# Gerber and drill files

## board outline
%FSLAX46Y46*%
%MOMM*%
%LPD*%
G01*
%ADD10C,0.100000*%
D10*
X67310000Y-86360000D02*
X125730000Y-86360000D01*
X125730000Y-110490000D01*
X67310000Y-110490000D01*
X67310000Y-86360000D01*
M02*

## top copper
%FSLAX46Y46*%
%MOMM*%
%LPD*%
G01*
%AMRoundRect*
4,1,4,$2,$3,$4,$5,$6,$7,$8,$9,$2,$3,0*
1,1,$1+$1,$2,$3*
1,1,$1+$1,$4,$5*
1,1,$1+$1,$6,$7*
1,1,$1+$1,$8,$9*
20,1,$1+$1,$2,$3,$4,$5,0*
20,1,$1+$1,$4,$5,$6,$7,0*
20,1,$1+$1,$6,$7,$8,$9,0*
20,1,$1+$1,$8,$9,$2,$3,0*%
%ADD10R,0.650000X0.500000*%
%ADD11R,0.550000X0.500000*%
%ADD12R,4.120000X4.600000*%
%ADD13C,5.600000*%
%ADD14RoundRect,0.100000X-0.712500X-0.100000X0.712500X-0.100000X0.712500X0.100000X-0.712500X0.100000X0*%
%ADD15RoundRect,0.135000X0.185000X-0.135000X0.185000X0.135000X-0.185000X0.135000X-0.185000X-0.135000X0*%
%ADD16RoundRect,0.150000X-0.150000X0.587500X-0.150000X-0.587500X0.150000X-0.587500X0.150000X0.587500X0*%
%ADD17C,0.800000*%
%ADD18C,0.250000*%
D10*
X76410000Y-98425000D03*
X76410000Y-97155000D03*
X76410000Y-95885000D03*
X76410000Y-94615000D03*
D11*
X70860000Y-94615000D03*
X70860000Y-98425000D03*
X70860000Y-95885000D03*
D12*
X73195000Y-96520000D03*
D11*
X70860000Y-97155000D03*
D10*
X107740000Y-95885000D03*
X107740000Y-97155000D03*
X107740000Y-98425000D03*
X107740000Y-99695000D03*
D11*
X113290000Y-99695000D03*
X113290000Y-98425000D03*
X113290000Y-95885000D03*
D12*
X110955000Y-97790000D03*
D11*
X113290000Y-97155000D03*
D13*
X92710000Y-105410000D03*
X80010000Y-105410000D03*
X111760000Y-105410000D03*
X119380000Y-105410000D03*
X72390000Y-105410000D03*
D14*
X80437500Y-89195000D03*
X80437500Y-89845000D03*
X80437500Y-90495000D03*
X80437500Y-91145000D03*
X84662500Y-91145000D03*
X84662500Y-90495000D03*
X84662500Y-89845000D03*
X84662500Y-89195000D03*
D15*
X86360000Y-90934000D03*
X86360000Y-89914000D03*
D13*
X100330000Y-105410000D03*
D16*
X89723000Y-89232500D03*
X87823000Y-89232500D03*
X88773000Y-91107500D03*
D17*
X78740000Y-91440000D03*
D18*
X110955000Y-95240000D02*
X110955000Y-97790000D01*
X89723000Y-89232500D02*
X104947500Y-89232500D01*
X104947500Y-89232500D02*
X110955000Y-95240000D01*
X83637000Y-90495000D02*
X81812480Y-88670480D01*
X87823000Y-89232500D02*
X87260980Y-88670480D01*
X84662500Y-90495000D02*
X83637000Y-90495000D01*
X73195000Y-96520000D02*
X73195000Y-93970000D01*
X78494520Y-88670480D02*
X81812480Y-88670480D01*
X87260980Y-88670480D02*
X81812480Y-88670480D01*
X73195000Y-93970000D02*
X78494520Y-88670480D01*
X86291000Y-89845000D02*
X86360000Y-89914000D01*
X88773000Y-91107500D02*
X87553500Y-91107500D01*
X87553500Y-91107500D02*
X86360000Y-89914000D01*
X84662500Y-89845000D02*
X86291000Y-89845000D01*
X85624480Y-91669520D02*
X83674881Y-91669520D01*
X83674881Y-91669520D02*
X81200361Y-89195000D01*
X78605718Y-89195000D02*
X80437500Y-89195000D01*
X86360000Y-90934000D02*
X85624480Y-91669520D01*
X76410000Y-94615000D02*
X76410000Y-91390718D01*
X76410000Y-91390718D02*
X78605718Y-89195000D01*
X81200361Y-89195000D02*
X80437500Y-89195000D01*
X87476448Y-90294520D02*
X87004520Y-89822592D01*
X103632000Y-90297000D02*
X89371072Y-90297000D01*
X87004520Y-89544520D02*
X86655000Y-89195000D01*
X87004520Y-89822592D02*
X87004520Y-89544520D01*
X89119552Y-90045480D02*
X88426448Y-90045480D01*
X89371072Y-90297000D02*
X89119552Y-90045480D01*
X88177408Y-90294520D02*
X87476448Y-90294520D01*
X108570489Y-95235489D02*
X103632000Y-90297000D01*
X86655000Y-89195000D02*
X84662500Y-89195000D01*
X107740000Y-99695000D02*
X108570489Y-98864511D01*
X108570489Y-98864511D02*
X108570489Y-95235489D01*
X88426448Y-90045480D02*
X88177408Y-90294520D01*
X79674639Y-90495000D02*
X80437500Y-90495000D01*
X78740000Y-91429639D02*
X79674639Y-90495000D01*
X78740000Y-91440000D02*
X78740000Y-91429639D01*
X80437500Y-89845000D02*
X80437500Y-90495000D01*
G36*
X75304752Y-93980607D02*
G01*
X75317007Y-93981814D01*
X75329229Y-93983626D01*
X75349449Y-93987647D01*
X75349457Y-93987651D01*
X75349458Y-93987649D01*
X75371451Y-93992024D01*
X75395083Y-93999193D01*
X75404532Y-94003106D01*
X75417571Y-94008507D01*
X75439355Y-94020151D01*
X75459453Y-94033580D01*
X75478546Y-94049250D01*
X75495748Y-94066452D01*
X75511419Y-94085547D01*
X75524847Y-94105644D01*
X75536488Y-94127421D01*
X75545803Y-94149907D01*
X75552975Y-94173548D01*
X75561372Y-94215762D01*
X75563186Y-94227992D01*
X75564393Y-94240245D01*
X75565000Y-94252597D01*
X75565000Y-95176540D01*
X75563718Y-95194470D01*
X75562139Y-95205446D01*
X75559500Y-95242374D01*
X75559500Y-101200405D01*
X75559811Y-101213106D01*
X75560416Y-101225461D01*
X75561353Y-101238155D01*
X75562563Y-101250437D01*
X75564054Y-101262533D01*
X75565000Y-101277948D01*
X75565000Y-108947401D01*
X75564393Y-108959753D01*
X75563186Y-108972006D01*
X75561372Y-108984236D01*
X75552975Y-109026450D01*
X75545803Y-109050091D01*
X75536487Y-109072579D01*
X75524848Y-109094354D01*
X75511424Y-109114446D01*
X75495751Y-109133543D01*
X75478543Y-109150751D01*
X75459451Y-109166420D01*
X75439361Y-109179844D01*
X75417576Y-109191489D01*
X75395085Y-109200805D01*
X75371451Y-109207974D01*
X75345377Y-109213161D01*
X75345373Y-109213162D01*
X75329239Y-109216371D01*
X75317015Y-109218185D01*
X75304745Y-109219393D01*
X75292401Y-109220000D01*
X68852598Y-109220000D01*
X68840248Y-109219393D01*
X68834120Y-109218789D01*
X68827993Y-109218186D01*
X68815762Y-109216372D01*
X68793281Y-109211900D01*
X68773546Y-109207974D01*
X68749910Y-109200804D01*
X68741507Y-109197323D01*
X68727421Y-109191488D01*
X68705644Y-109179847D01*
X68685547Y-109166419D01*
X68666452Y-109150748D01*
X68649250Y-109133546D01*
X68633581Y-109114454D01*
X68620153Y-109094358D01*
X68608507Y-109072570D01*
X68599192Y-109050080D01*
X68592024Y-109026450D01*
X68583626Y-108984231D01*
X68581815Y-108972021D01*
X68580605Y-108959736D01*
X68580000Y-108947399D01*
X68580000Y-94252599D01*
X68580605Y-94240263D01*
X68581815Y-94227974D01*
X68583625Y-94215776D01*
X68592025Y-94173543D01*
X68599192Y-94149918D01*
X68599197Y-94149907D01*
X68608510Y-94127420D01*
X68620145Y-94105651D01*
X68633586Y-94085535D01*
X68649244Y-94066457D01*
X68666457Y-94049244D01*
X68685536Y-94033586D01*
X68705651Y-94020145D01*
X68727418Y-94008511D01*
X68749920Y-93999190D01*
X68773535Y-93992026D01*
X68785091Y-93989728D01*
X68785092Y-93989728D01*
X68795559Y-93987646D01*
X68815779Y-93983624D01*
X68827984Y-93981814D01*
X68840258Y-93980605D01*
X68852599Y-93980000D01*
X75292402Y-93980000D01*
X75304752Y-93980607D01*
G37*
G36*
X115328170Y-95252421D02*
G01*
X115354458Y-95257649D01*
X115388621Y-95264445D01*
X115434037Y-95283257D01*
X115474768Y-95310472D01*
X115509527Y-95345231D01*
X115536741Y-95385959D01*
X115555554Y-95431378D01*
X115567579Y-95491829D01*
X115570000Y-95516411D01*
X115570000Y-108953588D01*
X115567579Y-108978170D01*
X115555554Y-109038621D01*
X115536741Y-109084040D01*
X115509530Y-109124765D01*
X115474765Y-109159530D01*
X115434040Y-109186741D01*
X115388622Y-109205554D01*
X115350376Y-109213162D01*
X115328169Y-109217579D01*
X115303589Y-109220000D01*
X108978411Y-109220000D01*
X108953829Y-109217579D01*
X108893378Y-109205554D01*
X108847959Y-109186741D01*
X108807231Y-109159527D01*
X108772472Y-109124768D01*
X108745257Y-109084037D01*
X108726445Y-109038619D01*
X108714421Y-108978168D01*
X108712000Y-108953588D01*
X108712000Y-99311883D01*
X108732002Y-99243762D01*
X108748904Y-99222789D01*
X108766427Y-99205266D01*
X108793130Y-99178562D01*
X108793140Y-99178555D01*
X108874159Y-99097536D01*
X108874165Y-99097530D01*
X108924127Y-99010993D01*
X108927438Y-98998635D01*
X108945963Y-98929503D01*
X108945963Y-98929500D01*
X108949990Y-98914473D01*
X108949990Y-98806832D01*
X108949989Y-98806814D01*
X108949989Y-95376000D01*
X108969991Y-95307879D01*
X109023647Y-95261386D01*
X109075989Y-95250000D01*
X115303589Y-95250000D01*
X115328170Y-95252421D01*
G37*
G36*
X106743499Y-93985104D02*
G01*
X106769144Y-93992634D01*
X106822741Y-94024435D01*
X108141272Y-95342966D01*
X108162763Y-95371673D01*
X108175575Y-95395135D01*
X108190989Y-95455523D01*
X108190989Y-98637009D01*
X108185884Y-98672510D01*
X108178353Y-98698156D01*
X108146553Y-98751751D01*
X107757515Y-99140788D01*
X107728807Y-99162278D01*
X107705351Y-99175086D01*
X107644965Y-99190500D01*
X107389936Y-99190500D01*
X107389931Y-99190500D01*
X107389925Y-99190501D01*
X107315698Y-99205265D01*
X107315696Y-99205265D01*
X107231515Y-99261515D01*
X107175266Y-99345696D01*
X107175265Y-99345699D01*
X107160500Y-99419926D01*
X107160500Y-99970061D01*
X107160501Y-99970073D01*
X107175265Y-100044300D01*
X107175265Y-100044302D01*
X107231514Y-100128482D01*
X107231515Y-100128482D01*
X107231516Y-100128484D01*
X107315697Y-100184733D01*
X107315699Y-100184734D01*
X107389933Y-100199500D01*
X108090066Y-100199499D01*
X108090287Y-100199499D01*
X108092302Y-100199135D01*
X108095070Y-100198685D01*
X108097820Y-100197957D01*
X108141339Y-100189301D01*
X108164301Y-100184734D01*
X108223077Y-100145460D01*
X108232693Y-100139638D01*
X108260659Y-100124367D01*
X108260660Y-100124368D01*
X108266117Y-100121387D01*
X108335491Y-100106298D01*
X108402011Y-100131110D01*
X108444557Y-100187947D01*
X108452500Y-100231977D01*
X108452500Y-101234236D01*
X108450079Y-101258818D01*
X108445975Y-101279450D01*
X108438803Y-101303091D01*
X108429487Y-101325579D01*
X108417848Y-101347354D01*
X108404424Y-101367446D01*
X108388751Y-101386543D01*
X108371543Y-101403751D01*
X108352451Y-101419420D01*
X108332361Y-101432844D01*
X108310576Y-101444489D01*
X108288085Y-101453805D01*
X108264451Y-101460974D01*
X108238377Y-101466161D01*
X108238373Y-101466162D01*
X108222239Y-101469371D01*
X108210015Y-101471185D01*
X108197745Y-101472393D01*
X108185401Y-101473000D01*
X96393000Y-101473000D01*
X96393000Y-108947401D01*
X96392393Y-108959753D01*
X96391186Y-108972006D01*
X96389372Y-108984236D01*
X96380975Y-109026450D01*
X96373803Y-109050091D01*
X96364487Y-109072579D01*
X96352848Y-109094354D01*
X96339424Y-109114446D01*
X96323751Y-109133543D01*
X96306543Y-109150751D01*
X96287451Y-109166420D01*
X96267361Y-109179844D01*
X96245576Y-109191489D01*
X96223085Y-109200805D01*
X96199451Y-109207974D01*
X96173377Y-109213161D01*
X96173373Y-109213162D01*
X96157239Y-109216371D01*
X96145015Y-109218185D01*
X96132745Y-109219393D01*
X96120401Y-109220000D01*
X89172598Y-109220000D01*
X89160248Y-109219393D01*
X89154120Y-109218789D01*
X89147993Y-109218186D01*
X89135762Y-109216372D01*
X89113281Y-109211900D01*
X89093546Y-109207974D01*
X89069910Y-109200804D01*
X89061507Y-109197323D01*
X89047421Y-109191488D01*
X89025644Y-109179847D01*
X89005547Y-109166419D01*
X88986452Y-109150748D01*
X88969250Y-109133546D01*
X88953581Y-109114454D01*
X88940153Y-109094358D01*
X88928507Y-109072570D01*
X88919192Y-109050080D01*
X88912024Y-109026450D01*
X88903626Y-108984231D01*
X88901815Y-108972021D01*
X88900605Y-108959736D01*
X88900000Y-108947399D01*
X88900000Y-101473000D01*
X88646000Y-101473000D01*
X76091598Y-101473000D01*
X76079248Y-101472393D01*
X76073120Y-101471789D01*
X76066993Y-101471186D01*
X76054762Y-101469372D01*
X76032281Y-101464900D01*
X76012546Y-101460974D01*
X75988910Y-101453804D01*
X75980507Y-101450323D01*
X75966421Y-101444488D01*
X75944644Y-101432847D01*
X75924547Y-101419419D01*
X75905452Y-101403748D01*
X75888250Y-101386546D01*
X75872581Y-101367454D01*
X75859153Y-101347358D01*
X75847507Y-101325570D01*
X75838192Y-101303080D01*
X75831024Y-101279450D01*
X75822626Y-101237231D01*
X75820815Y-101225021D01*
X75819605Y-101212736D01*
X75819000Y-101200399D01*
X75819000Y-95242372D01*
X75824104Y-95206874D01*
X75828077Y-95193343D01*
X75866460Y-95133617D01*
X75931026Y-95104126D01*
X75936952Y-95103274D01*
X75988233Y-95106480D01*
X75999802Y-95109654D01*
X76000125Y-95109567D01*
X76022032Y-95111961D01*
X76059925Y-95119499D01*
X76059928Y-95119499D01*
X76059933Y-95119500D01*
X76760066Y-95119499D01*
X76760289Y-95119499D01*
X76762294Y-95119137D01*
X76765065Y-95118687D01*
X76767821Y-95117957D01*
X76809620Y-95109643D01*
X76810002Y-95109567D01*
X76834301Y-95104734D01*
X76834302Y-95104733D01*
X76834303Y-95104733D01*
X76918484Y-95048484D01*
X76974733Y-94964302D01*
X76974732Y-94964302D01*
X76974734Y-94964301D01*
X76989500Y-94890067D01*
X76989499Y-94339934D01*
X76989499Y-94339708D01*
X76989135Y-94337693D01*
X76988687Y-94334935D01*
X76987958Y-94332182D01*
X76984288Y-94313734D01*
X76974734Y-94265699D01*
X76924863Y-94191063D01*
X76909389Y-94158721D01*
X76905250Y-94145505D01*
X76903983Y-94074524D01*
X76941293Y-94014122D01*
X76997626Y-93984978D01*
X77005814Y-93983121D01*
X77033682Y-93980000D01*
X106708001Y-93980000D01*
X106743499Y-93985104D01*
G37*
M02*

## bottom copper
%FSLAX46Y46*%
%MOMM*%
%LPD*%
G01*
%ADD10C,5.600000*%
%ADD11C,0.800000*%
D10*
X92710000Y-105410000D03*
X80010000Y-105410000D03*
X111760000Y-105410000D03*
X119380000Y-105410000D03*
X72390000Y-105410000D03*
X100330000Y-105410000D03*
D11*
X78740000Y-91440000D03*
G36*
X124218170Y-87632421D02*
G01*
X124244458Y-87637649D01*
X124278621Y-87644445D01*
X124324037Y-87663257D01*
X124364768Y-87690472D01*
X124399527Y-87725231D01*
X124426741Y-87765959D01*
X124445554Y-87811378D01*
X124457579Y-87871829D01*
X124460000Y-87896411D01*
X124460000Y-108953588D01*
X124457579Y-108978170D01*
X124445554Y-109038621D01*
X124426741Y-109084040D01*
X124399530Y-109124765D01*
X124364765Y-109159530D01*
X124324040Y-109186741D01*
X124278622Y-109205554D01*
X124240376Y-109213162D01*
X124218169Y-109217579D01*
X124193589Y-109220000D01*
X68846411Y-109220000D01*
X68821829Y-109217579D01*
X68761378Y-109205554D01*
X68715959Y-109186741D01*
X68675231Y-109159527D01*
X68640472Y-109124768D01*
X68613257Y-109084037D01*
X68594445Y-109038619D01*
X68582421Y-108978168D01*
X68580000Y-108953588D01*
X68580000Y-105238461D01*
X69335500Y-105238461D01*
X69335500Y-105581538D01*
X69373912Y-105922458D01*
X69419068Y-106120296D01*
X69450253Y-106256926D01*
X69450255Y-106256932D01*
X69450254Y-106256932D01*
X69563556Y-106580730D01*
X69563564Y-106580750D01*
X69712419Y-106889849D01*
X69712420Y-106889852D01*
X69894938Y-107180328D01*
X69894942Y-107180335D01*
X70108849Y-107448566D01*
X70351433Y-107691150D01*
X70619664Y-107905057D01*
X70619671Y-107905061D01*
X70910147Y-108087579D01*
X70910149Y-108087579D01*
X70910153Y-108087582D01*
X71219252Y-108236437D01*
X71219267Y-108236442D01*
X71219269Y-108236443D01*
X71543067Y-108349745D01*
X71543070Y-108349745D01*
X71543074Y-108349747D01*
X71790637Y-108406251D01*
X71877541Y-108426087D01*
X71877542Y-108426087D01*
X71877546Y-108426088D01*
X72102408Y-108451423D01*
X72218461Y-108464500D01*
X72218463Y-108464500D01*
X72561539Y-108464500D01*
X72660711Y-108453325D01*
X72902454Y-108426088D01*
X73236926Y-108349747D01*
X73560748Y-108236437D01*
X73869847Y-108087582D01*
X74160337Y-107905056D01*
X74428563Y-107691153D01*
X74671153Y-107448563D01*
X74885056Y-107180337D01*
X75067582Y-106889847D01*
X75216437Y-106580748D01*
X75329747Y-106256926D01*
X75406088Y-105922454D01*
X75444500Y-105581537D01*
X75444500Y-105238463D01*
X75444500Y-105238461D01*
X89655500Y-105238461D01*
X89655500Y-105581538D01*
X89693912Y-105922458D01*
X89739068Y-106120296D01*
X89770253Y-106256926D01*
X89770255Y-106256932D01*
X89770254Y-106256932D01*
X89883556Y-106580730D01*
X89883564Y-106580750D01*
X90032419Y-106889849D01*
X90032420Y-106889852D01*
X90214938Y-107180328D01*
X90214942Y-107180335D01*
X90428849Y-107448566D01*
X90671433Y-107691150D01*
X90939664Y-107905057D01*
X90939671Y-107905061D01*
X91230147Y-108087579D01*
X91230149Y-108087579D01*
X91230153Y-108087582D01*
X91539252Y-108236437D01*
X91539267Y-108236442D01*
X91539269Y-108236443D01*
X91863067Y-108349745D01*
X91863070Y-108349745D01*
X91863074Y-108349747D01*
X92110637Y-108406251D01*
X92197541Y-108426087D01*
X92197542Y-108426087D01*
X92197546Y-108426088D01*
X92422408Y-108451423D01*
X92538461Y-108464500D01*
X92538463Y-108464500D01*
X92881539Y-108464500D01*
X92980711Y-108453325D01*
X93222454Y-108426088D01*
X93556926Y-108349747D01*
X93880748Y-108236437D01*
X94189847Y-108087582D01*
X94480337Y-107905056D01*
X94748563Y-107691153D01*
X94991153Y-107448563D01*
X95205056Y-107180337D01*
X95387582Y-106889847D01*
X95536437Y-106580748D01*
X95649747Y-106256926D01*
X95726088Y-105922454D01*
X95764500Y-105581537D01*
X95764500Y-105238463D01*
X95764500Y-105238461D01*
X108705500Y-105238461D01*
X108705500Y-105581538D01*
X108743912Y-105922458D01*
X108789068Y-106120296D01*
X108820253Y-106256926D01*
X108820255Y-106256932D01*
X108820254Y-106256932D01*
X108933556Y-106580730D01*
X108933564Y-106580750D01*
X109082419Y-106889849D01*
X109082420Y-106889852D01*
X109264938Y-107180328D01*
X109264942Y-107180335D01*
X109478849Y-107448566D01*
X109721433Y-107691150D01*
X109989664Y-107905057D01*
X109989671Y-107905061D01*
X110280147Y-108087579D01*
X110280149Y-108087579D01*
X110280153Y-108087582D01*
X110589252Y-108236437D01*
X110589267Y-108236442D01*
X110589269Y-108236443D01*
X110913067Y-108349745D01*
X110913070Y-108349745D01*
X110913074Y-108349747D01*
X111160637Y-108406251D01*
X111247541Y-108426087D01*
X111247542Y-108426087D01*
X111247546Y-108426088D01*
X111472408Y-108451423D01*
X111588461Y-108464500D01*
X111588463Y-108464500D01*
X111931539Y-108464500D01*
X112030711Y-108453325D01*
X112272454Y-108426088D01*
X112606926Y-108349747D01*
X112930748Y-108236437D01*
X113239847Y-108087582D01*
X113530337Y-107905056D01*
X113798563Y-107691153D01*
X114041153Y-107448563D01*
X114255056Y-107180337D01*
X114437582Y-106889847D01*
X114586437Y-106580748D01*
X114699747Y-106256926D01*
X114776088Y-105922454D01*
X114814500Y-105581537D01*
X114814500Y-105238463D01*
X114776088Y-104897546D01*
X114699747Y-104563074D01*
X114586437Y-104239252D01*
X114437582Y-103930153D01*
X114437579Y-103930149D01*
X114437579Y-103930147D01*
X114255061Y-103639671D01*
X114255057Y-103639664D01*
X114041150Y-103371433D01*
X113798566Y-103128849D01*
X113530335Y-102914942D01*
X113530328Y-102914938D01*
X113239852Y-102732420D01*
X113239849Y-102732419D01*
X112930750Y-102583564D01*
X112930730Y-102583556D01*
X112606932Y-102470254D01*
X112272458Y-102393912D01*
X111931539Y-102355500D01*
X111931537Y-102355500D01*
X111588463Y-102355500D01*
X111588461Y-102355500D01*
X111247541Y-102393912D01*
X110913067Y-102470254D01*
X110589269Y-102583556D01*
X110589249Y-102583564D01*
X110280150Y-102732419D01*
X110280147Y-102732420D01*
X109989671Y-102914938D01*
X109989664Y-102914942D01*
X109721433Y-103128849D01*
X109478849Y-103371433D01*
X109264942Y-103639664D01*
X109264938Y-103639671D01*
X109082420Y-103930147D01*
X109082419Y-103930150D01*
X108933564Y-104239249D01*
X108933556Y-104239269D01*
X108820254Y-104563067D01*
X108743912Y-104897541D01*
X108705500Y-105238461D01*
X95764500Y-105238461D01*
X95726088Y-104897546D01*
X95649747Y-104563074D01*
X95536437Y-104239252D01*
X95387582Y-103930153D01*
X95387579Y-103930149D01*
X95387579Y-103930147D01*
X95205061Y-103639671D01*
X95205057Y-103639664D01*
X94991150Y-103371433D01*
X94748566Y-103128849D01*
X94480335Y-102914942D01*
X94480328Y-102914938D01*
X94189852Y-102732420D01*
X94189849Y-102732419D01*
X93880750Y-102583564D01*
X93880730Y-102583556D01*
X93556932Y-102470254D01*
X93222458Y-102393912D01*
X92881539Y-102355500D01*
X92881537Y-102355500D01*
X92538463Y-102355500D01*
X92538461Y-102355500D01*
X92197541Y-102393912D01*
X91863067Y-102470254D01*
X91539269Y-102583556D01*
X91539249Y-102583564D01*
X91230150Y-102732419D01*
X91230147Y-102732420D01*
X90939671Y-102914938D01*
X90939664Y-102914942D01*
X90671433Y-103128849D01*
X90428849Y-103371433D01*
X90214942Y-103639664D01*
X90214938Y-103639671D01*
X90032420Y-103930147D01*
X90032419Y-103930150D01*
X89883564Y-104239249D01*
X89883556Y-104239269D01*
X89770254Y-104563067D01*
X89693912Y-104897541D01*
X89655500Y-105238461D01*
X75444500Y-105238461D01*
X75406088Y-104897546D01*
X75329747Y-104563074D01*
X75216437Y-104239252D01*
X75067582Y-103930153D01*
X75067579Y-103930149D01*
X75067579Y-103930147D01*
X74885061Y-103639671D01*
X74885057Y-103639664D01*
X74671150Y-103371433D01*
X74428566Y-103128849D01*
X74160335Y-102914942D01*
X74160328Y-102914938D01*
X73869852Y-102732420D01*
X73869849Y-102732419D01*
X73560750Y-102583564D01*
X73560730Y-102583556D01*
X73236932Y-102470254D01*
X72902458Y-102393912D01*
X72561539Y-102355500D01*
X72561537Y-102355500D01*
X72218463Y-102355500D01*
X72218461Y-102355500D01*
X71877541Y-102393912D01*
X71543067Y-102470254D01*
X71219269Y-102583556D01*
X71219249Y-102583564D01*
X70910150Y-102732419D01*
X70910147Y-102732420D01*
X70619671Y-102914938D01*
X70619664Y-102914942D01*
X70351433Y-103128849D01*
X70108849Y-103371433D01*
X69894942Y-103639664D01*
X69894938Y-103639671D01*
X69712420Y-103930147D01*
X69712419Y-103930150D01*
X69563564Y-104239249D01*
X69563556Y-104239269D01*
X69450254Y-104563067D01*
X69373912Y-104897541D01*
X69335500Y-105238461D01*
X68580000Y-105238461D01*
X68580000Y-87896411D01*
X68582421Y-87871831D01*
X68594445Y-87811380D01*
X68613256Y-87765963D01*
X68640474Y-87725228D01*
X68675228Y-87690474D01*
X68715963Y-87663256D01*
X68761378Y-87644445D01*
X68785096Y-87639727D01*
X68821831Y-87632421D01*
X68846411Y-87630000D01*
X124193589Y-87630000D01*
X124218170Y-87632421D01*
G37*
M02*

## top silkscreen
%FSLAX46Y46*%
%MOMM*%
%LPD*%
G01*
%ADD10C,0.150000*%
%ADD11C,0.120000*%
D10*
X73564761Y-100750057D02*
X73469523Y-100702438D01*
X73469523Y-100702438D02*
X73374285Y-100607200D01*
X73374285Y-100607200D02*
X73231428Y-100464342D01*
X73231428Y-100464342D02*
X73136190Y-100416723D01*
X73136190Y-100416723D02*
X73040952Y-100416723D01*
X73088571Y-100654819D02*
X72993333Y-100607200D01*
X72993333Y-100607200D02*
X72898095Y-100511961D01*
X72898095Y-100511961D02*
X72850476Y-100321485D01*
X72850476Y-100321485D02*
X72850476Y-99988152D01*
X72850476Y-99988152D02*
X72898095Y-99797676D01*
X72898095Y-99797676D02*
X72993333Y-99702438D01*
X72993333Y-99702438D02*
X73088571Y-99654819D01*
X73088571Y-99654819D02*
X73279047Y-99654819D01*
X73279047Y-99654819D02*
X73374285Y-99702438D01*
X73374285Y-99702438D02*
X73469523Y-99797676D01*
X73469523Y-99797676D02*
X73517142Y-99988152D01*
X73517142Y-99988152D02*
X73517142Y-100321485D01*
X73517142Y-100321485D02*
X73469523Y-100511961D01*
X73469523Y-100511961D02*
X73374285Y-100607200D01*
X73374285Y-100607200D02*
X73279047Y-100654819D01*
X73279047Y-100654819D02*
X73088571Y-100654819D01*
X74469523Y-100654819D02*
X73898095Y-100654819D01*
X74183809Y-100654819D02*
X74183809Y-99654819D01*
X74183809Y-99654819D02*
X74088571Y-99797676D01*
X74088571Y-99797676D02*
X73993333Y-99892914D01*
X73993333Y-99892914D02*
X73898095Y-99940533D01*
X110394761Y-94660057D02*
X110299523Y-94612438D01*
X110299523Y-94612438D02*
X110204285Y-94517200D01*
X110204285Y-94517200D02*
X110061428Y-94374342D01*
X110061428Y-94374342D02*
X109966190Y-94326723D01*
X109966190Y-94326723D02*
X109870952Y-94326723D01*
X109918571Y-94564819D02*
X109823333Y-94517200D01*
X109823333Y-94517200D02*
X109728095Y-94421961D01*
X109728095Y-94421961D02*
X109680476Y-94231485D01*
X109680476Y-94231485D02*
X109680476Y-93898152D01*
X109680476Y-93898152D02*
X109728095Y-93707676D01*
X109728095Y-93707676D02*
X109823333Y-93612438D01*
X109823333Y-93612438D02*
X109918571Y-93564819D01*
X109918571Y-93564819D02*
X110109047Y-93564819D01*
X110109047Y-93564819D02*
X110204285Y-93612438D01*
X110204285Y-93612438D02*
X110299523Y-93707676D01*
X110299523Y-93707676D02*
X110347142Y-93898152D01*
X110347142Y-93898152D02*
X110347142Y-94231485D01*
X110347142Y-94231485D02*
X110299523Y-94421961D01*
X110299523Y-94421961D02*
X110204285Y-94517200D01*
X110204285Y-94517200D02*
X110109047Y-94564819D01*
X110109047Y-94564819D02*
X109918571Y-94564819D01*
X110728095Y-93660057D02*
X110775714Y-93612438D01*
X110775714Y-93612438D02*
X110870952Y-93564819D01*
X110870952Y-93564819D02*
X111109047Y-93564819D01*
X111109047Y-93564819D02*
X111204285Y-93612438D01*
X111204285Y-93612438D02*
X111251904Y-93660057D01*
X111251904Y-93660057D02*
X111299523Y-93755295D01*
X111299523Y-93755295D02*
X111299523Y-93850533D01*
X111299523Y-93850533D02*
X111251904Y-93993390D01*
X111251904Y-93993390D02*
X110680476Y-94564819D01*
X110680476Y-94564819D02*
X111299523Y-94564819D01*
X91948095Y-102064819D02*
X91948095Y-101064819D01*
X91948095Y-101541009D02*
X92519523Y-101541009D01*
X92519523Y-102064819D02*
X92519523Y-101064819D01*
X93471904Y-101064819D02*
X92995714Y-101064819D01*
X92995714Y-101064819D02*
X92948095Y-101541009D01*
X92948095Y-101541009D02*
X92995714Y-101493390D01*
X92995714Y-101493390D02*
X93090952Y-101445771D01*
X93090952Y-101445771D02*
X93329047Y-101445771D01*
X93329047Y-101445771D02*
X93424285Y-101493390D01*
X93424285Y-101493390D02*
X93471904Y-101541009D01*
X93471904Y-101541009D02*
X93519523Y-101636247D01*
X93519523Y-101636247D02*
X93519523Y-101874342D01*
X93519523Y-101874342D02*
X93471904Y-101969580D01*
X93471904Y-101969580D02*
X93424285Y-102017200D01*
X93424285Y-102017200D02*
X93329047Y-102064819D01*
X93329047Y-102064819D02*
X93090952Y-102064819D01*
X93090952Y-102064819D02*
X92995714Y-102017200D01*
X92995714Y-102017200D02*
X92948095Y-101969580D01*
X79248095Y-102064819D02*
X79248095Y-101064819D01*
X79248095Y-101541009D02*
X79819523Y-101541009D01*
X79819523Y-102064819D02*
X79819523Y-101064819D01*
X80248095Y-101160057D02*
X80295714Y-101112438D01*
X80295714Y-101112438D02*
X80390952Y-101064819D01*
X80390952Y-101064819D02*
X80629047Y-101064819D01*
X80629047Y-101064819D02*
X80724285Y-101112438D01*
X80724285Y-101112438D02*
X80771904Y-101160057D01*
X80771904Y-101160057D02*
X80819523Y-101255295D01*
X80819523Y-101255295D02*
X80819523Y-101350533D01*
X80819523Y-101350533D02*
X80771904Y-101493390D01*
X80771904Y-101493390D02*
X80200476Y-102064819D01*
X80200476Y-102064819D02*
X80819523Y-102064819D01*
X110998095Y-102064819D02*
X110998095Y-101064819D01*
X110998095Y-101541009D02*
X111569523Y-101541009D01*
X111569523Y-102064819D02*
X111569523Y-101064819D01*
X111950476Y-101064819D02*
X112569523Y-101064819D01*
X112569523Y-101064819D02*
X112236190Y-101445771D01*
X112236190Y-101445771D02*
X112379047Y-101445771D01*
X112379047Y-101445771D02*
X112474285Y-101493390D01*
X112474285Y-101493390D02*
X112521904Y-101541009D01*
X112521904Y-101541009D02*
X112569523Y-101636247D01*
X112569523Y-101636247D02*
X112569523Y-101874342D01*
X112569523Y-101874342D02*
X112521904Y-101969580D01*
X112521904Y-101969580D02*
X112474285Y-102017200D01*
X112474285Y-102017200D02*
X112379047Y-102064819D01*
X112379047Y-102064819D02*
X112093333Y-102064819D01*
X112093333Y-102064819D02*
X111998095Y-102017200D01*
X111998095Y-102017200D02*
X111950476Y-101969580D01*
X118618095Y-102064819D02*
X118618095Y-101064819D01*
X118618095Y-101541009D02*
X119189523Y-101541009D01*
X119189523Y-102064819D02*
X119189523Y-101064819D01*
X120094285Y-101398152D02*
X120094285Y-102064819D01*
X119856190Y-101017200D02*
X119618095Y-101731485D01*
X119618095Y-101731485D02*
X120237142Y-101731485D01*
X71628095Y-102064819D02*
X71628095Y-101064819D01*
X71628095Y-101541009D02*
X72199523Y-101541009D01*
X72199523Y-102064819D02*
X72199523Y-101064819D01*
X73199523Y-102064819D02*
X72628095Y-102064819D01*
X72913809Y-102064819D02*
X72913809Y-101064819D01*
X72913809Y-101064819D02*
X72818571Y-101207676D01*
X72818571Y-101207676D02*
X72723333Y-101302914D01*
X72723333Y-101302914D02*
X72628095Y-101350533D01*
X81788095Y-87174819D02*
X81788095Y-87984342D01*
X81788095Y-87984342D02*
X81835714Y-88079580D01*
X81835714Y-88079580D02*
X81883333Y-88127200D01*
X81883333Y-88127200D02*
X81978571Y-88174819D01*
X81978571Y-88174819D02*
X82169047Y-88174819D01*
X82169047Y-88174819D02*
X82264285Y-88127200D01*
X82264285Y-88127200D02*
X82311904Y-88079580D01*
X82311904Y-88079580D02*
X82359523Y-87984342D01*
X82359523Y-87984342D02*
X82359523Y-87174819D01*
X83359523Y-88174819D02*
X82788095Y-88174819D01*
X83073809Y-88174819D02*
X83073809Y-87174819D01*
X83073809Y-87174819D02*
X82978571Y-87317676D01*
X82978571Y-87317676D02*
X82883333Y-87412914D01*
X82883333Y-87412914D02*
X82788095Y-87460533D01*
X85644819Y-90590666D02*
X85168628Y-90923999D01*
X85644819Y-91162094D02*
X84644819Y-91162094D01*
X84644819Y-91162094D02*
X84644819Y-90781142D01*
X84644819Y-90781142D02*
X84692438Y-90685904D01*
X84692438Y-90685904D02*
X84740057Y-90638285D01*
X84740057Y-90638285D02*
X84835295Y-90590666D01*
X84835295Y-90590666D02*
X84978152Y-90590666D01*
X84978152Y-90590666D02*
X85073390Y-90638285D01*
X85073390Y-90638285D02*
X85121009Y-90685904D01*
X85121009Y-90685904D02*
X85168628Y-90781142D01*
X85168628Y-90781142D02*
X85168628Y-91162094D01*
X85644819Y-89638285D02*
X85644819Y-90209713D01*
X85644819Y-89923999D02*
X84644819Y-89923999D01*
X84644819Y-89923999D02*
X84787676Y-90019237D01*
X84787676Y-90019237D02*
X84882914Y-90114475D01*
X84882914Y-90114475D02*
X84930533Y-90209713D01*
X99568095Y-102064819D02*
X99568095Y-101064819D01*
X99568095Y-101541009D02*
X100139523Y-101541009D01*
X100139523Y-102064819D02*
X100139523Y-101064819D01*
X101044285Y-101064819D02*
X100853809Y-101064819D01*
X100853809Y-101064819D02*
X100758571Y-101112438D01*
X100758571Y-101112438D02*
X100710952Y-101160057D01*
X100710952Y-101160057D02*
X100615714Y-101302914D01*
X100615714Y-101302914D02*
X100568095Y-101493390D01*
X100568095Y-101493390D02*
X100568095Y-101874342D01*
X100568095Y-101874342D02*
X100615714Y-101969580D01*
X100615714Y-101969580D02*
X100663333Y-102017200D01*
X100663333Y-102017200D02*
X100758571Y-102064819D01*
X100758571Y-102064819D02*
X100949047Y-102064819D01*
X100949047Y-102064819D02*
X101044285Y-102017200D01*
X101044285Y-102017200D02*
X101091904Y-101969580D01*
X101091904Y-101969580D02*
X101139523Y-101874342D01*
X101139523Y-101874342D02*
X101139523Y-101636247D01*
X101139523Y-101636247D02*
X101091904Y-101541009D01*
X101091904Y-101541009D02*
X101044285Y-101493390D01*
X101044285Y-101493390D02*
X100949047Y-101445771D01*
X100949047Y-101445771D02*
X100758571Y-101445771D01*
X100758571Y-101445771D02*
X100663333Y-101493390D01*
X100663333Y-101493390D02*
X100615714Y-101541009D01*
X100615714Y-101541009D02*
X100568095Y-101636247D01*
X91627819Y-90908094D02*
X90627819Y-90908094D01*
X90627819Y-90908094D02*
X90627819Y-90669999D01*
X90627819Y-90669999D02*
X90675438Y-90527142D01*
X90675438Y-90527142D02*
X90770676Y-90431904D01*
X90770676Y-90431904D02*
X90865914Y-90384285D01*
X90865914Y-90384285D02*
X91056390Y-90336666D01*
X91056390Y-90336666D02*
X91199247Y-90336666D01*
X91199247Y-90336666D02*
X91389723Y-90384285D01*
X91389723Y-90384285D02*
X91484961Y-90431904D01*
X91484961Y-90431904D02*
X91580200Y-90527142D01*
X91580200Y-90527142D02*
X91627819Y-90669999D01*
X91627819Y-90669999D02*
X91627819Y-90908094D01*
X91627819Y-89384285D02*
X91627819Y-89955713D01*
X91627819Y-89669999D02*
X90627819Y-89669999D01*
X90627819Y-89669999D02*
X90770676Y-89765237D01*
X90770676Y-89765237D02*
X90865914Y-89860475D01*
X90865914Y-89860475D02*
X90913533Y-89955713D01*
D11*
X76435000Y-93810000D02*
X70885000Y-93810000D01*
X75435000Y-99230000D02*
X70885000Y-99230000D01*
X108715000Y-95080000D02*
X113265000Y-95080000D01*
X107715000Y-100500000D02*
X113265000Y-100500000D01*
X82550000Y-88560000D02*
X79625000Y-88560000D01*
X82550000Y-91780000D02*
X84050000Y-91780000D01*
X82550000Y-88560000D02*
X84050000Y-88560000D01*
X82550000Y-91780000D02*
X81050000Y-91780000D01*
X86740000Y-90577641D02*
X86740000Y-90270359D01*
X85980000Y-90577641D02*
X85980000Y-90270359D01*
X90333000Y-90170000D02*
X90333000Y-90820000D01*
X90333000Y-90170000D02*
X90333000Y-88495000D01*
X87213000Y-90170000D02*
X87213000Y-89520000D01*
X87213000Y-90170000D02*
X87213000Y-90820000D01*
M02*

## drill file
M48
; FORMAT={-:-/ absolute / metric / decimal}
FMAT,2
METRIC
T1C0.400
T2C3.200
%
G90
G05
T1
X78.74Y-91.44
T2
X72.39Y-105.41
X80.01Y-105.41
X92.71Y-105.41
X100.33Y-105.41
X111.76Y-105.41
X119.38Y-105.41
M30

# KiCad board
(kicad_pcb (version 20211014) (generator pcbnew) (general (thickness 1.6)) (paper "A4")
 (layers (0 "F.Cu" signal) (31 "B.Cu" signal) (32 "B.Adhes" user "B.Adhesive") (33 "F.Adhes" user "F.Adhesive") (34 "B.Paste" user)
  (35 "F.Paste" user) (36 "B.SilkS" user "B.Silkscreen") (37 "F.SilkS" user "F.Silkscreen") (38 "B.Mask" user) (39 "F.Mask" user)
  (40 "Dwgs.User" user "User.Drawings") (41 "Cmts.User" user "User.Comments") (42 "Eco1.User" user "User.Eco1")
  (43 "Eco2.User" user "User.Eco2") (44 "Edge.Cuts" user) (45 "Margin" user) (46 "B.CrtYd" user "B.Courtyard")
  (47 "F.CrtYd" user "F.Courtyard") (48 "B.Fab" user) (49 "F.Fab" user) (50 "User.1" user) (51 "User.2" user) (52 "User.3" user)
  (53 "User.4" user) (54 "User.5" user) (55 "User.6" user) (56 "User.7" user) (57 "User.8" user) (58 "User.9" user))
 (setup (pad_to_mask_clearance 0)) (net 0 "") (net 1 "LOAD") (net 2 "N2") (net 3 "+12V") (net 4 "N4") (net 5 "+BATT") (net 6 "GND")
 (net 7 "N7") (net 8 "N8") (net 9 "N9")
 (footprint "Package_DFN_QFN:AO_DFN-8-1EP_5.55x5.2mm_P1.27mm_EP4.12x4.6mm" (layer "F.Cu") (at 73.66 96.52 180)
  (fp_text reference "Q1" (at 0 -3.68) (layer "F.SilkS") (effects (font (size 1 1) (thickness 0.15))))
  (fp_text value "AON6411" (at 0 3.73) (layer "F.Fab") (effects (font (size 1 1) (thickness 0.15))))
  (fp_line (start -2.775 2.71) (end 2.775 2.71) (layer "F.SilkS") (width 0.12))
  (fp_line (start -1.775 -2.71) (end 2.775 -2.71) (layer "F.SilkS") (width 0.12))
  (pad "" smd rect (at -0.02 -1.65 90) (size 0.9 0.78) (layers "F.Paste"))
  (pad "" smd rect (at 0.96 1.65 90) (size 0.9 0.78) (layers "F.Paste"))
  (pad "" smd rect (at 0.96 0.55 90) (size 0.9 0.78) (layers "F.Paste"))
  (pad "" smd rect (at 1.94 -0.55 90) (size 0.9 0.78) (layers "F.Paste"))
  (pad "" smd rect (at 1.94 -1.65 90) (size 0.9 0.78) (layers "F.Paste"))
  (pad "" smd rect (at -1 1.65 90) (size 0.9 0.78) (layers "F.Paste"))
  (pad "" smd rect (at 0.96 -0.55 90) (size 0.9 0.78) (layers "F.Paste"))
  (pad "" smd rect (at -1 -0.55 90) (size 0.9 0.78) (layers "F.Paste"))
  (pad "" smd rect (at -1 0.55 90) (size 0.9 0.78) (layers "F.Paste"))
  (pad "" smd rect (at 1.94 0.55 90) (size 0.9 0.78) (layers "F.Paste"))
  (pad "" smd rect (at -0.02 1.65 90) (size 0.9 0.78) (layers "F.Paste"))
  (pad "" smd rect (at -0.02 -0.55 90) (size 0.9 0.78) (layers "F.Paste"))
  (pad "" smd rect (at 0.96 -1.65 90) (size 0.9 0.78) (layers "F.Paste"))
  (pad "" smd rect (at -1 -1.65 90) (size 0.9 0.78) (layers "F.Paste"))
  (pad "" smd rect (at 1.94 1.65 90) (size 0.9 0.78) (layers "F.Paste"))
  (pad "" smd rect (at -0.02 0.55 90) (size 0.9 0.78) (layers "F.Paste"))
  (pad "1" smd rect (at -2.75 -1.905 90) (size 0.5 0.65) (layers "F.Cu" "F.Paste" "F.Mask") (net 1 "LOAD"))
  (pad "2" smd rect (at -2.75 -0.635 90) (size 0.5 0.65) (layers "F.Cu" "F.Paste" "F.Mask") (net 1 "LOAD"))
  (pad "3" smd rect (at -2.75 0.635 90) (size 0.5 0.65) (layers "F.Cu" "F.Paste" "F.Mask") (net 1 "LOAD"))
  (pad "4" smd rect (at -2.75 1.905 90) (size 0.5 0.65) (layers "F.Cu" "F.Paste" "F.Mask") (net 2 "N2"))
  (pad "5" smd rect (at 2.8 1.905 90) (size 0.5 0.55) (layers "F.Cu" "F.Paste" "F.Mask") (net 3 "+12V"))
  (pad "5" smd rect (at 2.8 -1.905 90) (size 0.5 0.55) (layers "F.Cu" "F.Paste" "F.Mask") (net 3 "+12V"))
  (pad "5" smd rect (at 2.8 0.635 90) (size 0.5 0.55) (layers "F.Cu" "F.Paste" "F.Mask") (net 3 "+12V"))
  (pad "5" smd rect (at 0.465 0 90) (size 4.6 4.12) (layers "F.Cu" "F.Mask") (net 3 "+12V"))
  (pad "5" smd rect (at 2.8 -0.635 90) (size 0.5 0.55) (layers "F.Cu" "F.Paste" "F.Mask") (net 3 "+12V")))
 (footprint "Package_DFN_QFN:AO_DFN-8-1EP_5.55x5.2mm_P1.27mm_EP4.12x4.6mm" (layer "F.Cu") (at 110.49 97.79)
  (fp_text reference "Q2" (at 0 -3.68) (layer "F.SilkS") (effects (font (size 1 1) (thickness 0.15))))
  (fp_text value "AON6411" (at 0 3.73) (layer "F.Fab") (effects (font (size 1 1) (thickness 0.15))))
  (fp_line (start -1.775 -2.71) (end 2.775 -2.71) (layer "F.SilkS") (width 0.12))
  (fp_line (start -2.775 2.71) (end 2.775 2.71) (layer "F.SilkS") (width 0.12))
  (pad "" smd rect (at 1.94 1.65 270) (size 0.9 0.78) (layers "F.Paste"))
  (pad "" smd rect (at -0.02 1.65 270) (size 0.9 0.78) (layers "F.Paste"))
  (pad "" smd rect (at -1 -1.65 270) (size 0.9 0.78) (layers "F.Paste"))
  (pad "" smd rect (at -1 0.55 270) (size 0.9 0.78) (layers "F.Paste"))
  (pad "" smd rect (at 0.96 0.55 270) (size 0.9 0.78) (layers "F.Paste"))
  (pad "" smd rect (at 0.96 1.65 270) (size 0.9 0.78) (layers "F.Paste"))
  (pad "" smd rect (at 0.96 -1.65 270) (size 0.9 0.78) (layers "F.Paste"))
  (pad "" smd rect (at 0.96 -0.55 270) (size 0.9 0.78) (layers "F.Paste"))
  (pad "" smd rect (at 1.94 -1.65 270) (size 0.9 0.78) (layers "F.Paste"))
  (pad "" smd rect (at -0.02 -1.65 270) (size 0.9 0.78) (layers "F.Paste"))
  (pad "" smd rect (at -0.02 -0.55 270) (size 0.9 0.78) (layers "F.Paste"))
  (pad "" smd rect (at 1.94 0.55 270) (size 0.9 0.78) (layers "F.Paste"))
  (pad "" smd rect (at 1.94 -0.55 270) (size 0.9 0.78) (layers "F.Paste"))
  (pad "" smd rect (at -1 -0.55 270) (size 0.9 0.78) (layers "F.Paste"))
  (pad "" smd rect (at -0.02 0.55 270) (size 0.9 0.78) (layers "F.Paste"))
  (pad "" smd rect (at -1 1.65 270) (size 0.9 0.78) (layers "F.Paste"))
  (pad "1" smd rect (at -2.75 -1.905 270) (size 0.5 0.65) (layers "F.Cu" "F.Paste" "F.Mask") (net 1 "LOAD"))
  (pad "2" smd rect (at -2.75 -0.635 270) (size 0.5 0.65) (layers "F.Cu" "F.Paste" "F.Mask") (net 1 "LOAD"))
  (pad "3" smd rect (at -2.75 0.635 270) (size 0.5 0.65) (layers "F.Cu" "F.Paste" "F.Mask") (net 1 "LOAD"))
  (pad "4" smd rect (at -2.75 1.905 270) (size 0.5 0.65) (layers "F.Cu" "F.Paste" "F.Mask") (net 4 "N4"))
  (pad "5" smd rect (at 2.8 1.905 270) (size 0.5 0.55) (layers "F.Cu" "F.Paste" "F.Mask") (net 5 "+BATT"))
  (pad "5" smd rect (at 2.8 0.635 270) (size 0.5 0.55) (layers "F.Cu" "F.Paste" "F.Mask") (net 5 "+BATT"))
  (pad "5" smd rect (at 2.8 -1.905 270) (size 0.5 0.55) (layers "F.Cu" "F.Paste" "F.Mask") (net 5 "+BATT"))
  (pad "5" smd rect (at 0.465 0 270) (size 4.6 4.12) (layers "F.Cu" "F.Mask") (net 5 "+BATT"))
  (pad "5" smd rect (at 2.8 -0.635 270) (size 0.5 0.55) (layers "F.Cu" "F.Paste" "F.Mask") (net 5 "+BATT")))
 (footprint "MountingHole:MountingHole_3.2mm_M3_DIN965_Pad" (layer "F.Cu") (at 92.71 105.41)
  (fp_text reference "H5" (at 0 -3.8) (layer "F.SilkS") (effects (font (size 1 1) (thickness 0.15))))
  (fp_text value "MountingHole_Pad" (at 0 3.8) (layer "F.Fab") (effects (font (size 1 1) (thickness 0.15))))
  (pad "1" thru_hole circle (at 0 0) (size 5.6 5.6) (drill 3.2) (layers *.Cu *.Mask) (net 1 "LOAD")))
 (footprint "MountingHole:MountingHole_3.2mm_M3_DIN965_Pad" (layer "F.Cu") (at 80.01 105.41)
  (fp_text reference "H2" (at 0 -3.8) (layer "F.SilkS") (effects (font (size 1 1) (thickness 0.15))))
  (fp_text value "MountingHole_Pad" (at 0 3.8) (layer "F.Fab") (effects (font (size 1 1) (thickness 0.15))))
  (pad "1" thru_hole circle (at 0 0) (size 5.6 5.6) (drill 3.2) (layers *.Cu *.Mask) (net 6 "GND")))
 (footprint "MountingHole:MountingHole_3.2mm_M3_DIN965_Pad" (layer "F.Cu") (at 111.76 105.41)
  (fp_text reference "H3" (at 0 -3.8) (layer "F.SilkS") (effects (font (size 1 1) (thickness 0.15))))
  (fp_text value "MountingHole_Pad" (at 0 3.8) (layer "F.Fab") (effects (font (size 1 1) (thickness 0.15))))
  (pad "1" thru_hole circle (at 0 0) (size 5.6 5.6) (drill 3.2) (layers *.Cu *.Mask) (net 5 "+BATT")))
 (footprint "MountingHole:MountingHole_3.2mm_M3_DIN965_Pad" (layer "F.Cu") (at 119.38 105.41)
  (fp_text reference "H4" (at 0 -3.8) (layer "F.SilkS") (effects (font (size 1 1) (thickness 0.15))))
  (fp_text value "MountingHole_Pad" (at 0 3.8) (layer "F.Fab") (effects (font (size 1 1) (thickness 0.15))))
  (pad "1" thru_hole circle (at 0 0) (size 5.6 5.6) (drill 3.2) (layers *.Cu *.Mask) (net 6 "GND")))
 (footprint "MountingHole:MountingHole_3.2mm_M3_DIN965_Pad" (layer "F.Cu") (at 72.39 105.41)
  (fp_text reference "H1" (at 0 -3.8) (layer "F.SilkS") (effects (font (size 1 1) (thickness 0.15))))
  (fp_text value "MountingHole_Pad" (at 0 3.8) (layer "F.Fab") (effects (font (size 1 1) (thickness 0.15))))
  (pad "1" thru_hole circle (at 0 0) (size 5.6 5.6) (drill 3.2) (layers *.Cu *.Mask) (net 3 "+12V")))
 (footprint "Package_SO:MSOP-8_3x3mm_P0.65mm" (layer "F.Cu") (at 82.55 90.17)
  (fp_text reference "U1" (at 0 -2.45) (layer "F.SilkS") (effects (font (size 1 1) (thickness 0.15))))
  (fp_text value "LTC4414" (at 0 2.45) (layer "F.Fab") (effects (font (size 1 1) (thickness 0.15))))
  (fp_line (start 0 -1.61) (end -2.925 -1.61) (layer "F.SilkS") (width 0.12))
  (fp_line (start 0 1.61) (end 1.5 1.61) (layer "F.SilkS") (width 0.12))
  (fp_line (start 0 -1.61) (end 1.5 -1.61) (layer "F.SilkS") (width 0.12))
  (fp_line (start 0 1.61) (end -1.5 1.61) (layer "F.SilkS") (width 0.12))
  (pad "1" smd roundrect (at -2.1125 -0.975) (size 1.625 0.4) (layers "F.Cu" "F.Paste" "F.Mask") (roundrect_rratio 0.25) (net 2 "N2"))
  (pad "2" smd roundrect (at -2.1125 -0.325) (size 1.625 0.4) (layers "F.Cu" "F.Paste" "F.Mask") (roundrect_rratio 0.25) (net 6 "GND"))
  (pad "3" smd roundrect (at -2.1125 0.325) (size 1.625 0.4) (layers "F.Cu" "F.Paste" "F.Mask") (roundrect_rratio 0.25) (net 6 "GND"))
  (pad "4" smd roundrect (at -2.1125 0.975) (size 1.625 0.4) (layers "F.Cu" "F.Paste" "F.Mask") (roundrect_rratio 0.25) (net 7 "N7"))
  (pad "5" smd roundrect (at 2.1125 0.975) (size 1.625 0.4) (layers "F.Cu" "F.Paste" "F.Mask") (roundrect_rratio 0.25) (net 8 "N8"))
  (pad "6" smd roundrect (at 2.1125 0.325) (size 1.625 0.4) (layers "F.Cu" "F.Paste" "F.Mask") (roundrect_rratio 0.25) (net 3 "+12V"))
  (pad "7" smd roundrect (at 2.1125 -0.325) (size 1.625 0.4) (layers "F.Cu" "F.Paste" "F.Mask") (roundrect_rratio 0.25) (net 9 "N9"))
  (pad "8" smd roundrect (at 2.1125 -0.975) (size 1.625 0.4) (layers "F.Cu" "F.Paste" "F.Mask") (roundrect_rratio 0.25) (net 4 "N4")))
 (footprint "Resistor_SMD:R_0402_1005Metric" (layer "F.Cu") (at 86.36 90.424 90)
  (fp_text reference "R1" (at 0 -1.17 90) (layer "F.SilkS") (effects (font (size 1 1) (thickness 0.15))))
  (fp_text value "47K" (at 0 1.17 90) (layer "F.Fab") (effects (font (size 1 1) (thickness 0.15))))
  (fp_line (start -0.153641 0.38) (end 0.153641 0.38) (layer "F.SilkS") (width 0.12))
  (fp_line (start -0.153641 -0.38) (end 0.153641 -0.38) (layer "F.SilkS") (width 0.12))
  (pad "1" smd roundrect (at -0.51 0 90) (size 0.54 0.64) (layers "F.Cu" "F.Paste" "F.Mask") (roundrect_rratio 0.25) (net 2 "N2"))
  (pad "2" smd roundrect (at 0.51 0 90) (size 0.54 0.64) (layers "F.Cu" "F.Paste" "F.Mask") (roundrect_rratio 0.25) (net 9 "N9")))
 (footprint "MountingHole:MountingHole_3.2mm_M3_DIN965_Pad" (layer "F.Cu") (at 100.33 105.41)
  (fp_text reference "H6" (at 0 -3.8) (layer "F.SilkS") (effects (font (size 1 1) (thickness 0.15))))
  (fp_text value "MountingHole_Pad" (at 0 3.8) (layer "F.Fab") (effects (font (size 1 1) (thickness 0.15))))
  (pad "1" thru_hole circle (at 0 0) (size 5.6 5.6) (drill 3.2) (layers *.Cu *.Mask) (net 6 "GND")))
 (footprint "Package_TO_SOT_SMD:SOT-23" (layer "F.Cu") (at 88.773 90.17 -90)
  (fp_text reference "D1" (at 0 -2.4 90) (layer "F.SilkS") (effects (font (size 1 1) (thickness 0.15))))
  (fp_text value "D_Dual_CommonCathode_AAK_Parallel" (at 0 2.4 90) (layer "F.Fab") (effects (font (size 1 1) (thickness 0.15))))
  (fp_line (start 0 -1.56) (end 0.65 -1.56) (layer "F.SilkS") (width 0.12))
  (fp_line (start 0 -1.56) (end -1.675 -1.56) (layer "F.SilkS") (width 0.12))
  (fp_line (start 0 1.56) (end -0.65 1.56) (layer "F.SilkS") (width 0.12))
  (fp_line (start 0 1.56) (end 0.65 1.56) (layer "F.SilkS") (width 0.12))
  (pad "1" smd roundrect (at -0.9375 -0.95 270) (size 1.475 0.6) (layers "F.Cu" "F.Paste" "F.Mask") (roundrect_rratio 0.25) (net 5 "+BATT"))
  (pad "2" smd roundrect (at -0.9375 0.95 270) (size 1.475 0.6) (layers "F.Cu" "F.Paste" "F.Mask") (roundrect_rratio 0.25) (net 3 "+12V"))
  (pad "3" smd roundrect (at 0.9375 0 270) (size 1.475 0.6) (layers "F.Cu" "F.Paste" "F.Mask") (roundrect_rratio 0.25) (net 9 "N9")))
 (gr_rect (start 67.31 86.36) (end 125.73 110.49) (layer "Edge.Cuts") (width 0.1) (fill none))
 (segment (start 110.955 95.24) (end 110.955 97.79) (width 0.25) (layer "F.Cu") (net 5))
 (segment (start 89.723 89.2325) (end 104.9475 89.2325) (width 0.25) (layer "F.Cu") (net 5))
 (segment (start 104.9475 89.2325) (end 110.955 95.24) (width 0.25) (layer "F.Cu") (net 5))
 (segment (start 83.637 90.495) (end 81.81248 88.67048) (width 0.25) (layer "F.Cu") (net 3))
 (segment (start 87.823 89.2325) (end 87.26098 88.67048) (width 0.25) (layer "F.Cu") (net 3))
 (segment (start 84.6625 90.495) (end 83.637 90.495) (width 0.25) (layer "F.Cu") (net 3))
 (segment (start 73.195 96.52) (end 73.195 93.97) (width 0.25) (layer "F.Cu") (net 3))
 (segment (start 78.49452 88.67048) (end 81.81248 88.67048) (width 0.25) (layer "F.Cu") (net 3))
 (segment (start 87.26098 88.67048) (end 81.81248 88.67048) (width 0.25) (layer "F.Cu") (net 3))
 (segment (start 73.195 93.97) (end 78.49452 88.67048) (width 0.25) (layer "F.Cu") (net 3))
 (segment (start 86.291 89.845) (end 86.36 89.914) (width 0.25) (layer "F.Cu") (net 9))
 (segment (start 88.773 91.1075) (end 87.5535 91.1075) (width 0.25) (layer "F.Cu") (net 9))
 (segment (start 87.5535 91.1075) (end 86.36 89.914) (width 0.25) (layer "F.Cu") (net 9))
 (segment (start 84.6625 89.845) (end 86.291 89.845) (width 0.25) (layer "F.Cu") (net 9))
 (segment (start 85.62448 91.66952) (end 83.674881 91.66952) (width 0.25) (layer "F.Cu") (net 2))
 (segment (start 83.674881 91.66952) (end 81.200361 89.195) (width 0.25) (layer "F.Cu") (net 2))
 (segment (start 78.605718 89.195) (end 80.4375 89.195) (width 0.25) (layer "F.Cu") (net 2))
 (segment (start 86.36 90.934) (end 85.62448 91.66952) (width 0.25) (layer "F.Cu") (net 2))
 (segment (start 76.41 94.615) (end 76.41 91.390718) (width 0.25) (layer "F.Cu") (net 2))
 (segment (start 76.41 91.390718) (end 78.605718 89.195) (width 0.25) (layer "F.Cu") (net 2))
 (segment (start 81.200361 89.195) (end 80.4375 89.195) (width 0.25) (layer "F.Cu") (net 2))
 (segment (start 87.476448 90.29452) (end 87.00452 89.822592) (width 0.25) (layer "F.Cu") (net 4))
 (segment (start 103.632 90.297) (end 89.371072 90.297) (width 0.25) (layer "F.Cu") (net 4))
 (segment (start 87.00452 89.54452) (end 86.655 89.195) (width 0.25) (layer "F.Cu") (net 4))
 (segment (start 87.00452 89.822592) (end 87.00452 89.54452) (width 0.25) (layer "F.Cu") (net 4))
 (segment (start 89.119552 90.04548) (end 88.426448 90.04548) (width 0.25) (layer "F.Cu") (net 4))
 (segment (start 89.371072 90.297) (end 89.119552 90.04548) (width 0.25) (layer "F.Cu") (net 4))
 (segment (start 88.177408 90.29452) (end 87.476448 90.29452) (width 0.25) (layer "F.Cu") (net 4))
 (segment (start 108.570489 95.235489) (end 103.632 90.297) (width 0.25) (layer "F.Cu") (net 4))
 (segment (start 86.655 89.195) (end 84.6625 89.195) (width 0.25) (layer "F.Cu") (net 4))
 (segment (start 107.74 99.695) (end 108.570489 98.864511) (width 0.25) (layer "F.Cu") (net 4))
 (segment (start 108.570489 98.864511) (end 108.570489 95.235489) (width 0.25) (layer "F.Cu") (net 4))
 (segment (start 88.426448 90.04548) (end 88.177408 90.29452) (width 0.25) (layer "F.Cu") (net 4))
 (segment (start 79.674639 90.495) (end 80.4375 90.495) (width 0.25) (layer "F.Cu") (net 6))
 (segment (start 78.74 91.429639) (end 79.674639 90.495) (width 0.25) (layer "F.Cu") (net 6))
 (segment (start 78.74 91.44) (end 78.74 91.429639) (width 0.25) (layer "F.Cu") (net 6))
 (segment (start 80.4375 89.845) (end 80.4375 90.495) (width 0.25) (layer "F.Cu") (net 6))
 (via (at 78.74 91.44) (size 0.8) (drill 0.4) (layers "F.Cu" "B.Cu") (free) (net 6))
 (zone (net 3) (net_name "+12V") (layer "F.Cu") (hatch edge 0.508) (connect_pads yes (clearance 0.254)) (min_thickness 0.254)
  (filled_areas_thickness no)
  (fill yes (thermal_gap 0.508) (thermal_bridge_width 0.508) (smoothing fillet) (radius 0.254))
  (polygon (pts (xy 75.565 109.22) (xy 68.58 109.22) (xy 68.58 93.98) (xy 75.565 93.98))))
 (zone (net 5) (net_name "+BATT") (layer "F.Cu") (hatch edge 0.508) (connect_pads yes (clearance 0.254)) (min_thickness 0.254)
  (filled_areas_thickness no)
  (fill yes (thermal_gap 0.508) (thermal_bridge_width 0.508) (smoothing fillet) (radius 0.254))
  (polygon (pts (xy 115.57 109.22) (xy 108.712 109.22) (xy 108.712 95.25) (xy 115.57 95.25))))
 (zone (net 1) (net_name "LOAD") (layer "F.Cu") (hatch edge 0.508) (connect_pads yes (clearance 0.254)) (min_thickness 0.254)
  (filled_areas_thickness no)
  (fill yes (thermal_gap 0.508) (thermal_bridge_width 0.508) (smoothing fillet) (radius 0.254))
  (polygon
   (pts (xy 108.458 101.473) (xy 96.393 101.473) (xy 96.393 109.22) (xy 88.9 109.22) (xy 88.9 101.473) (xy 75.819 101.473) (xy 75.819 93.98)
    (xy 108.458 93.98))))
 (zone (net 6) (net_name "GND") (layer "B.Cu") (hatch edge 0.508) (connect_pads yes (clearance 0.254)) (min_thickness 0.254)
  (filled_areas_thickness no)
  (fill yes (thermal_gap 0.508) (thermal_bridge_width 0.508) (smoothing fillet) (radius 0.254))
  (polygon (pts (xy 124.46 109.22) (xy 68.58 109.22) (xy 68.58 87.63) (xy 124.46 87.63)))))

